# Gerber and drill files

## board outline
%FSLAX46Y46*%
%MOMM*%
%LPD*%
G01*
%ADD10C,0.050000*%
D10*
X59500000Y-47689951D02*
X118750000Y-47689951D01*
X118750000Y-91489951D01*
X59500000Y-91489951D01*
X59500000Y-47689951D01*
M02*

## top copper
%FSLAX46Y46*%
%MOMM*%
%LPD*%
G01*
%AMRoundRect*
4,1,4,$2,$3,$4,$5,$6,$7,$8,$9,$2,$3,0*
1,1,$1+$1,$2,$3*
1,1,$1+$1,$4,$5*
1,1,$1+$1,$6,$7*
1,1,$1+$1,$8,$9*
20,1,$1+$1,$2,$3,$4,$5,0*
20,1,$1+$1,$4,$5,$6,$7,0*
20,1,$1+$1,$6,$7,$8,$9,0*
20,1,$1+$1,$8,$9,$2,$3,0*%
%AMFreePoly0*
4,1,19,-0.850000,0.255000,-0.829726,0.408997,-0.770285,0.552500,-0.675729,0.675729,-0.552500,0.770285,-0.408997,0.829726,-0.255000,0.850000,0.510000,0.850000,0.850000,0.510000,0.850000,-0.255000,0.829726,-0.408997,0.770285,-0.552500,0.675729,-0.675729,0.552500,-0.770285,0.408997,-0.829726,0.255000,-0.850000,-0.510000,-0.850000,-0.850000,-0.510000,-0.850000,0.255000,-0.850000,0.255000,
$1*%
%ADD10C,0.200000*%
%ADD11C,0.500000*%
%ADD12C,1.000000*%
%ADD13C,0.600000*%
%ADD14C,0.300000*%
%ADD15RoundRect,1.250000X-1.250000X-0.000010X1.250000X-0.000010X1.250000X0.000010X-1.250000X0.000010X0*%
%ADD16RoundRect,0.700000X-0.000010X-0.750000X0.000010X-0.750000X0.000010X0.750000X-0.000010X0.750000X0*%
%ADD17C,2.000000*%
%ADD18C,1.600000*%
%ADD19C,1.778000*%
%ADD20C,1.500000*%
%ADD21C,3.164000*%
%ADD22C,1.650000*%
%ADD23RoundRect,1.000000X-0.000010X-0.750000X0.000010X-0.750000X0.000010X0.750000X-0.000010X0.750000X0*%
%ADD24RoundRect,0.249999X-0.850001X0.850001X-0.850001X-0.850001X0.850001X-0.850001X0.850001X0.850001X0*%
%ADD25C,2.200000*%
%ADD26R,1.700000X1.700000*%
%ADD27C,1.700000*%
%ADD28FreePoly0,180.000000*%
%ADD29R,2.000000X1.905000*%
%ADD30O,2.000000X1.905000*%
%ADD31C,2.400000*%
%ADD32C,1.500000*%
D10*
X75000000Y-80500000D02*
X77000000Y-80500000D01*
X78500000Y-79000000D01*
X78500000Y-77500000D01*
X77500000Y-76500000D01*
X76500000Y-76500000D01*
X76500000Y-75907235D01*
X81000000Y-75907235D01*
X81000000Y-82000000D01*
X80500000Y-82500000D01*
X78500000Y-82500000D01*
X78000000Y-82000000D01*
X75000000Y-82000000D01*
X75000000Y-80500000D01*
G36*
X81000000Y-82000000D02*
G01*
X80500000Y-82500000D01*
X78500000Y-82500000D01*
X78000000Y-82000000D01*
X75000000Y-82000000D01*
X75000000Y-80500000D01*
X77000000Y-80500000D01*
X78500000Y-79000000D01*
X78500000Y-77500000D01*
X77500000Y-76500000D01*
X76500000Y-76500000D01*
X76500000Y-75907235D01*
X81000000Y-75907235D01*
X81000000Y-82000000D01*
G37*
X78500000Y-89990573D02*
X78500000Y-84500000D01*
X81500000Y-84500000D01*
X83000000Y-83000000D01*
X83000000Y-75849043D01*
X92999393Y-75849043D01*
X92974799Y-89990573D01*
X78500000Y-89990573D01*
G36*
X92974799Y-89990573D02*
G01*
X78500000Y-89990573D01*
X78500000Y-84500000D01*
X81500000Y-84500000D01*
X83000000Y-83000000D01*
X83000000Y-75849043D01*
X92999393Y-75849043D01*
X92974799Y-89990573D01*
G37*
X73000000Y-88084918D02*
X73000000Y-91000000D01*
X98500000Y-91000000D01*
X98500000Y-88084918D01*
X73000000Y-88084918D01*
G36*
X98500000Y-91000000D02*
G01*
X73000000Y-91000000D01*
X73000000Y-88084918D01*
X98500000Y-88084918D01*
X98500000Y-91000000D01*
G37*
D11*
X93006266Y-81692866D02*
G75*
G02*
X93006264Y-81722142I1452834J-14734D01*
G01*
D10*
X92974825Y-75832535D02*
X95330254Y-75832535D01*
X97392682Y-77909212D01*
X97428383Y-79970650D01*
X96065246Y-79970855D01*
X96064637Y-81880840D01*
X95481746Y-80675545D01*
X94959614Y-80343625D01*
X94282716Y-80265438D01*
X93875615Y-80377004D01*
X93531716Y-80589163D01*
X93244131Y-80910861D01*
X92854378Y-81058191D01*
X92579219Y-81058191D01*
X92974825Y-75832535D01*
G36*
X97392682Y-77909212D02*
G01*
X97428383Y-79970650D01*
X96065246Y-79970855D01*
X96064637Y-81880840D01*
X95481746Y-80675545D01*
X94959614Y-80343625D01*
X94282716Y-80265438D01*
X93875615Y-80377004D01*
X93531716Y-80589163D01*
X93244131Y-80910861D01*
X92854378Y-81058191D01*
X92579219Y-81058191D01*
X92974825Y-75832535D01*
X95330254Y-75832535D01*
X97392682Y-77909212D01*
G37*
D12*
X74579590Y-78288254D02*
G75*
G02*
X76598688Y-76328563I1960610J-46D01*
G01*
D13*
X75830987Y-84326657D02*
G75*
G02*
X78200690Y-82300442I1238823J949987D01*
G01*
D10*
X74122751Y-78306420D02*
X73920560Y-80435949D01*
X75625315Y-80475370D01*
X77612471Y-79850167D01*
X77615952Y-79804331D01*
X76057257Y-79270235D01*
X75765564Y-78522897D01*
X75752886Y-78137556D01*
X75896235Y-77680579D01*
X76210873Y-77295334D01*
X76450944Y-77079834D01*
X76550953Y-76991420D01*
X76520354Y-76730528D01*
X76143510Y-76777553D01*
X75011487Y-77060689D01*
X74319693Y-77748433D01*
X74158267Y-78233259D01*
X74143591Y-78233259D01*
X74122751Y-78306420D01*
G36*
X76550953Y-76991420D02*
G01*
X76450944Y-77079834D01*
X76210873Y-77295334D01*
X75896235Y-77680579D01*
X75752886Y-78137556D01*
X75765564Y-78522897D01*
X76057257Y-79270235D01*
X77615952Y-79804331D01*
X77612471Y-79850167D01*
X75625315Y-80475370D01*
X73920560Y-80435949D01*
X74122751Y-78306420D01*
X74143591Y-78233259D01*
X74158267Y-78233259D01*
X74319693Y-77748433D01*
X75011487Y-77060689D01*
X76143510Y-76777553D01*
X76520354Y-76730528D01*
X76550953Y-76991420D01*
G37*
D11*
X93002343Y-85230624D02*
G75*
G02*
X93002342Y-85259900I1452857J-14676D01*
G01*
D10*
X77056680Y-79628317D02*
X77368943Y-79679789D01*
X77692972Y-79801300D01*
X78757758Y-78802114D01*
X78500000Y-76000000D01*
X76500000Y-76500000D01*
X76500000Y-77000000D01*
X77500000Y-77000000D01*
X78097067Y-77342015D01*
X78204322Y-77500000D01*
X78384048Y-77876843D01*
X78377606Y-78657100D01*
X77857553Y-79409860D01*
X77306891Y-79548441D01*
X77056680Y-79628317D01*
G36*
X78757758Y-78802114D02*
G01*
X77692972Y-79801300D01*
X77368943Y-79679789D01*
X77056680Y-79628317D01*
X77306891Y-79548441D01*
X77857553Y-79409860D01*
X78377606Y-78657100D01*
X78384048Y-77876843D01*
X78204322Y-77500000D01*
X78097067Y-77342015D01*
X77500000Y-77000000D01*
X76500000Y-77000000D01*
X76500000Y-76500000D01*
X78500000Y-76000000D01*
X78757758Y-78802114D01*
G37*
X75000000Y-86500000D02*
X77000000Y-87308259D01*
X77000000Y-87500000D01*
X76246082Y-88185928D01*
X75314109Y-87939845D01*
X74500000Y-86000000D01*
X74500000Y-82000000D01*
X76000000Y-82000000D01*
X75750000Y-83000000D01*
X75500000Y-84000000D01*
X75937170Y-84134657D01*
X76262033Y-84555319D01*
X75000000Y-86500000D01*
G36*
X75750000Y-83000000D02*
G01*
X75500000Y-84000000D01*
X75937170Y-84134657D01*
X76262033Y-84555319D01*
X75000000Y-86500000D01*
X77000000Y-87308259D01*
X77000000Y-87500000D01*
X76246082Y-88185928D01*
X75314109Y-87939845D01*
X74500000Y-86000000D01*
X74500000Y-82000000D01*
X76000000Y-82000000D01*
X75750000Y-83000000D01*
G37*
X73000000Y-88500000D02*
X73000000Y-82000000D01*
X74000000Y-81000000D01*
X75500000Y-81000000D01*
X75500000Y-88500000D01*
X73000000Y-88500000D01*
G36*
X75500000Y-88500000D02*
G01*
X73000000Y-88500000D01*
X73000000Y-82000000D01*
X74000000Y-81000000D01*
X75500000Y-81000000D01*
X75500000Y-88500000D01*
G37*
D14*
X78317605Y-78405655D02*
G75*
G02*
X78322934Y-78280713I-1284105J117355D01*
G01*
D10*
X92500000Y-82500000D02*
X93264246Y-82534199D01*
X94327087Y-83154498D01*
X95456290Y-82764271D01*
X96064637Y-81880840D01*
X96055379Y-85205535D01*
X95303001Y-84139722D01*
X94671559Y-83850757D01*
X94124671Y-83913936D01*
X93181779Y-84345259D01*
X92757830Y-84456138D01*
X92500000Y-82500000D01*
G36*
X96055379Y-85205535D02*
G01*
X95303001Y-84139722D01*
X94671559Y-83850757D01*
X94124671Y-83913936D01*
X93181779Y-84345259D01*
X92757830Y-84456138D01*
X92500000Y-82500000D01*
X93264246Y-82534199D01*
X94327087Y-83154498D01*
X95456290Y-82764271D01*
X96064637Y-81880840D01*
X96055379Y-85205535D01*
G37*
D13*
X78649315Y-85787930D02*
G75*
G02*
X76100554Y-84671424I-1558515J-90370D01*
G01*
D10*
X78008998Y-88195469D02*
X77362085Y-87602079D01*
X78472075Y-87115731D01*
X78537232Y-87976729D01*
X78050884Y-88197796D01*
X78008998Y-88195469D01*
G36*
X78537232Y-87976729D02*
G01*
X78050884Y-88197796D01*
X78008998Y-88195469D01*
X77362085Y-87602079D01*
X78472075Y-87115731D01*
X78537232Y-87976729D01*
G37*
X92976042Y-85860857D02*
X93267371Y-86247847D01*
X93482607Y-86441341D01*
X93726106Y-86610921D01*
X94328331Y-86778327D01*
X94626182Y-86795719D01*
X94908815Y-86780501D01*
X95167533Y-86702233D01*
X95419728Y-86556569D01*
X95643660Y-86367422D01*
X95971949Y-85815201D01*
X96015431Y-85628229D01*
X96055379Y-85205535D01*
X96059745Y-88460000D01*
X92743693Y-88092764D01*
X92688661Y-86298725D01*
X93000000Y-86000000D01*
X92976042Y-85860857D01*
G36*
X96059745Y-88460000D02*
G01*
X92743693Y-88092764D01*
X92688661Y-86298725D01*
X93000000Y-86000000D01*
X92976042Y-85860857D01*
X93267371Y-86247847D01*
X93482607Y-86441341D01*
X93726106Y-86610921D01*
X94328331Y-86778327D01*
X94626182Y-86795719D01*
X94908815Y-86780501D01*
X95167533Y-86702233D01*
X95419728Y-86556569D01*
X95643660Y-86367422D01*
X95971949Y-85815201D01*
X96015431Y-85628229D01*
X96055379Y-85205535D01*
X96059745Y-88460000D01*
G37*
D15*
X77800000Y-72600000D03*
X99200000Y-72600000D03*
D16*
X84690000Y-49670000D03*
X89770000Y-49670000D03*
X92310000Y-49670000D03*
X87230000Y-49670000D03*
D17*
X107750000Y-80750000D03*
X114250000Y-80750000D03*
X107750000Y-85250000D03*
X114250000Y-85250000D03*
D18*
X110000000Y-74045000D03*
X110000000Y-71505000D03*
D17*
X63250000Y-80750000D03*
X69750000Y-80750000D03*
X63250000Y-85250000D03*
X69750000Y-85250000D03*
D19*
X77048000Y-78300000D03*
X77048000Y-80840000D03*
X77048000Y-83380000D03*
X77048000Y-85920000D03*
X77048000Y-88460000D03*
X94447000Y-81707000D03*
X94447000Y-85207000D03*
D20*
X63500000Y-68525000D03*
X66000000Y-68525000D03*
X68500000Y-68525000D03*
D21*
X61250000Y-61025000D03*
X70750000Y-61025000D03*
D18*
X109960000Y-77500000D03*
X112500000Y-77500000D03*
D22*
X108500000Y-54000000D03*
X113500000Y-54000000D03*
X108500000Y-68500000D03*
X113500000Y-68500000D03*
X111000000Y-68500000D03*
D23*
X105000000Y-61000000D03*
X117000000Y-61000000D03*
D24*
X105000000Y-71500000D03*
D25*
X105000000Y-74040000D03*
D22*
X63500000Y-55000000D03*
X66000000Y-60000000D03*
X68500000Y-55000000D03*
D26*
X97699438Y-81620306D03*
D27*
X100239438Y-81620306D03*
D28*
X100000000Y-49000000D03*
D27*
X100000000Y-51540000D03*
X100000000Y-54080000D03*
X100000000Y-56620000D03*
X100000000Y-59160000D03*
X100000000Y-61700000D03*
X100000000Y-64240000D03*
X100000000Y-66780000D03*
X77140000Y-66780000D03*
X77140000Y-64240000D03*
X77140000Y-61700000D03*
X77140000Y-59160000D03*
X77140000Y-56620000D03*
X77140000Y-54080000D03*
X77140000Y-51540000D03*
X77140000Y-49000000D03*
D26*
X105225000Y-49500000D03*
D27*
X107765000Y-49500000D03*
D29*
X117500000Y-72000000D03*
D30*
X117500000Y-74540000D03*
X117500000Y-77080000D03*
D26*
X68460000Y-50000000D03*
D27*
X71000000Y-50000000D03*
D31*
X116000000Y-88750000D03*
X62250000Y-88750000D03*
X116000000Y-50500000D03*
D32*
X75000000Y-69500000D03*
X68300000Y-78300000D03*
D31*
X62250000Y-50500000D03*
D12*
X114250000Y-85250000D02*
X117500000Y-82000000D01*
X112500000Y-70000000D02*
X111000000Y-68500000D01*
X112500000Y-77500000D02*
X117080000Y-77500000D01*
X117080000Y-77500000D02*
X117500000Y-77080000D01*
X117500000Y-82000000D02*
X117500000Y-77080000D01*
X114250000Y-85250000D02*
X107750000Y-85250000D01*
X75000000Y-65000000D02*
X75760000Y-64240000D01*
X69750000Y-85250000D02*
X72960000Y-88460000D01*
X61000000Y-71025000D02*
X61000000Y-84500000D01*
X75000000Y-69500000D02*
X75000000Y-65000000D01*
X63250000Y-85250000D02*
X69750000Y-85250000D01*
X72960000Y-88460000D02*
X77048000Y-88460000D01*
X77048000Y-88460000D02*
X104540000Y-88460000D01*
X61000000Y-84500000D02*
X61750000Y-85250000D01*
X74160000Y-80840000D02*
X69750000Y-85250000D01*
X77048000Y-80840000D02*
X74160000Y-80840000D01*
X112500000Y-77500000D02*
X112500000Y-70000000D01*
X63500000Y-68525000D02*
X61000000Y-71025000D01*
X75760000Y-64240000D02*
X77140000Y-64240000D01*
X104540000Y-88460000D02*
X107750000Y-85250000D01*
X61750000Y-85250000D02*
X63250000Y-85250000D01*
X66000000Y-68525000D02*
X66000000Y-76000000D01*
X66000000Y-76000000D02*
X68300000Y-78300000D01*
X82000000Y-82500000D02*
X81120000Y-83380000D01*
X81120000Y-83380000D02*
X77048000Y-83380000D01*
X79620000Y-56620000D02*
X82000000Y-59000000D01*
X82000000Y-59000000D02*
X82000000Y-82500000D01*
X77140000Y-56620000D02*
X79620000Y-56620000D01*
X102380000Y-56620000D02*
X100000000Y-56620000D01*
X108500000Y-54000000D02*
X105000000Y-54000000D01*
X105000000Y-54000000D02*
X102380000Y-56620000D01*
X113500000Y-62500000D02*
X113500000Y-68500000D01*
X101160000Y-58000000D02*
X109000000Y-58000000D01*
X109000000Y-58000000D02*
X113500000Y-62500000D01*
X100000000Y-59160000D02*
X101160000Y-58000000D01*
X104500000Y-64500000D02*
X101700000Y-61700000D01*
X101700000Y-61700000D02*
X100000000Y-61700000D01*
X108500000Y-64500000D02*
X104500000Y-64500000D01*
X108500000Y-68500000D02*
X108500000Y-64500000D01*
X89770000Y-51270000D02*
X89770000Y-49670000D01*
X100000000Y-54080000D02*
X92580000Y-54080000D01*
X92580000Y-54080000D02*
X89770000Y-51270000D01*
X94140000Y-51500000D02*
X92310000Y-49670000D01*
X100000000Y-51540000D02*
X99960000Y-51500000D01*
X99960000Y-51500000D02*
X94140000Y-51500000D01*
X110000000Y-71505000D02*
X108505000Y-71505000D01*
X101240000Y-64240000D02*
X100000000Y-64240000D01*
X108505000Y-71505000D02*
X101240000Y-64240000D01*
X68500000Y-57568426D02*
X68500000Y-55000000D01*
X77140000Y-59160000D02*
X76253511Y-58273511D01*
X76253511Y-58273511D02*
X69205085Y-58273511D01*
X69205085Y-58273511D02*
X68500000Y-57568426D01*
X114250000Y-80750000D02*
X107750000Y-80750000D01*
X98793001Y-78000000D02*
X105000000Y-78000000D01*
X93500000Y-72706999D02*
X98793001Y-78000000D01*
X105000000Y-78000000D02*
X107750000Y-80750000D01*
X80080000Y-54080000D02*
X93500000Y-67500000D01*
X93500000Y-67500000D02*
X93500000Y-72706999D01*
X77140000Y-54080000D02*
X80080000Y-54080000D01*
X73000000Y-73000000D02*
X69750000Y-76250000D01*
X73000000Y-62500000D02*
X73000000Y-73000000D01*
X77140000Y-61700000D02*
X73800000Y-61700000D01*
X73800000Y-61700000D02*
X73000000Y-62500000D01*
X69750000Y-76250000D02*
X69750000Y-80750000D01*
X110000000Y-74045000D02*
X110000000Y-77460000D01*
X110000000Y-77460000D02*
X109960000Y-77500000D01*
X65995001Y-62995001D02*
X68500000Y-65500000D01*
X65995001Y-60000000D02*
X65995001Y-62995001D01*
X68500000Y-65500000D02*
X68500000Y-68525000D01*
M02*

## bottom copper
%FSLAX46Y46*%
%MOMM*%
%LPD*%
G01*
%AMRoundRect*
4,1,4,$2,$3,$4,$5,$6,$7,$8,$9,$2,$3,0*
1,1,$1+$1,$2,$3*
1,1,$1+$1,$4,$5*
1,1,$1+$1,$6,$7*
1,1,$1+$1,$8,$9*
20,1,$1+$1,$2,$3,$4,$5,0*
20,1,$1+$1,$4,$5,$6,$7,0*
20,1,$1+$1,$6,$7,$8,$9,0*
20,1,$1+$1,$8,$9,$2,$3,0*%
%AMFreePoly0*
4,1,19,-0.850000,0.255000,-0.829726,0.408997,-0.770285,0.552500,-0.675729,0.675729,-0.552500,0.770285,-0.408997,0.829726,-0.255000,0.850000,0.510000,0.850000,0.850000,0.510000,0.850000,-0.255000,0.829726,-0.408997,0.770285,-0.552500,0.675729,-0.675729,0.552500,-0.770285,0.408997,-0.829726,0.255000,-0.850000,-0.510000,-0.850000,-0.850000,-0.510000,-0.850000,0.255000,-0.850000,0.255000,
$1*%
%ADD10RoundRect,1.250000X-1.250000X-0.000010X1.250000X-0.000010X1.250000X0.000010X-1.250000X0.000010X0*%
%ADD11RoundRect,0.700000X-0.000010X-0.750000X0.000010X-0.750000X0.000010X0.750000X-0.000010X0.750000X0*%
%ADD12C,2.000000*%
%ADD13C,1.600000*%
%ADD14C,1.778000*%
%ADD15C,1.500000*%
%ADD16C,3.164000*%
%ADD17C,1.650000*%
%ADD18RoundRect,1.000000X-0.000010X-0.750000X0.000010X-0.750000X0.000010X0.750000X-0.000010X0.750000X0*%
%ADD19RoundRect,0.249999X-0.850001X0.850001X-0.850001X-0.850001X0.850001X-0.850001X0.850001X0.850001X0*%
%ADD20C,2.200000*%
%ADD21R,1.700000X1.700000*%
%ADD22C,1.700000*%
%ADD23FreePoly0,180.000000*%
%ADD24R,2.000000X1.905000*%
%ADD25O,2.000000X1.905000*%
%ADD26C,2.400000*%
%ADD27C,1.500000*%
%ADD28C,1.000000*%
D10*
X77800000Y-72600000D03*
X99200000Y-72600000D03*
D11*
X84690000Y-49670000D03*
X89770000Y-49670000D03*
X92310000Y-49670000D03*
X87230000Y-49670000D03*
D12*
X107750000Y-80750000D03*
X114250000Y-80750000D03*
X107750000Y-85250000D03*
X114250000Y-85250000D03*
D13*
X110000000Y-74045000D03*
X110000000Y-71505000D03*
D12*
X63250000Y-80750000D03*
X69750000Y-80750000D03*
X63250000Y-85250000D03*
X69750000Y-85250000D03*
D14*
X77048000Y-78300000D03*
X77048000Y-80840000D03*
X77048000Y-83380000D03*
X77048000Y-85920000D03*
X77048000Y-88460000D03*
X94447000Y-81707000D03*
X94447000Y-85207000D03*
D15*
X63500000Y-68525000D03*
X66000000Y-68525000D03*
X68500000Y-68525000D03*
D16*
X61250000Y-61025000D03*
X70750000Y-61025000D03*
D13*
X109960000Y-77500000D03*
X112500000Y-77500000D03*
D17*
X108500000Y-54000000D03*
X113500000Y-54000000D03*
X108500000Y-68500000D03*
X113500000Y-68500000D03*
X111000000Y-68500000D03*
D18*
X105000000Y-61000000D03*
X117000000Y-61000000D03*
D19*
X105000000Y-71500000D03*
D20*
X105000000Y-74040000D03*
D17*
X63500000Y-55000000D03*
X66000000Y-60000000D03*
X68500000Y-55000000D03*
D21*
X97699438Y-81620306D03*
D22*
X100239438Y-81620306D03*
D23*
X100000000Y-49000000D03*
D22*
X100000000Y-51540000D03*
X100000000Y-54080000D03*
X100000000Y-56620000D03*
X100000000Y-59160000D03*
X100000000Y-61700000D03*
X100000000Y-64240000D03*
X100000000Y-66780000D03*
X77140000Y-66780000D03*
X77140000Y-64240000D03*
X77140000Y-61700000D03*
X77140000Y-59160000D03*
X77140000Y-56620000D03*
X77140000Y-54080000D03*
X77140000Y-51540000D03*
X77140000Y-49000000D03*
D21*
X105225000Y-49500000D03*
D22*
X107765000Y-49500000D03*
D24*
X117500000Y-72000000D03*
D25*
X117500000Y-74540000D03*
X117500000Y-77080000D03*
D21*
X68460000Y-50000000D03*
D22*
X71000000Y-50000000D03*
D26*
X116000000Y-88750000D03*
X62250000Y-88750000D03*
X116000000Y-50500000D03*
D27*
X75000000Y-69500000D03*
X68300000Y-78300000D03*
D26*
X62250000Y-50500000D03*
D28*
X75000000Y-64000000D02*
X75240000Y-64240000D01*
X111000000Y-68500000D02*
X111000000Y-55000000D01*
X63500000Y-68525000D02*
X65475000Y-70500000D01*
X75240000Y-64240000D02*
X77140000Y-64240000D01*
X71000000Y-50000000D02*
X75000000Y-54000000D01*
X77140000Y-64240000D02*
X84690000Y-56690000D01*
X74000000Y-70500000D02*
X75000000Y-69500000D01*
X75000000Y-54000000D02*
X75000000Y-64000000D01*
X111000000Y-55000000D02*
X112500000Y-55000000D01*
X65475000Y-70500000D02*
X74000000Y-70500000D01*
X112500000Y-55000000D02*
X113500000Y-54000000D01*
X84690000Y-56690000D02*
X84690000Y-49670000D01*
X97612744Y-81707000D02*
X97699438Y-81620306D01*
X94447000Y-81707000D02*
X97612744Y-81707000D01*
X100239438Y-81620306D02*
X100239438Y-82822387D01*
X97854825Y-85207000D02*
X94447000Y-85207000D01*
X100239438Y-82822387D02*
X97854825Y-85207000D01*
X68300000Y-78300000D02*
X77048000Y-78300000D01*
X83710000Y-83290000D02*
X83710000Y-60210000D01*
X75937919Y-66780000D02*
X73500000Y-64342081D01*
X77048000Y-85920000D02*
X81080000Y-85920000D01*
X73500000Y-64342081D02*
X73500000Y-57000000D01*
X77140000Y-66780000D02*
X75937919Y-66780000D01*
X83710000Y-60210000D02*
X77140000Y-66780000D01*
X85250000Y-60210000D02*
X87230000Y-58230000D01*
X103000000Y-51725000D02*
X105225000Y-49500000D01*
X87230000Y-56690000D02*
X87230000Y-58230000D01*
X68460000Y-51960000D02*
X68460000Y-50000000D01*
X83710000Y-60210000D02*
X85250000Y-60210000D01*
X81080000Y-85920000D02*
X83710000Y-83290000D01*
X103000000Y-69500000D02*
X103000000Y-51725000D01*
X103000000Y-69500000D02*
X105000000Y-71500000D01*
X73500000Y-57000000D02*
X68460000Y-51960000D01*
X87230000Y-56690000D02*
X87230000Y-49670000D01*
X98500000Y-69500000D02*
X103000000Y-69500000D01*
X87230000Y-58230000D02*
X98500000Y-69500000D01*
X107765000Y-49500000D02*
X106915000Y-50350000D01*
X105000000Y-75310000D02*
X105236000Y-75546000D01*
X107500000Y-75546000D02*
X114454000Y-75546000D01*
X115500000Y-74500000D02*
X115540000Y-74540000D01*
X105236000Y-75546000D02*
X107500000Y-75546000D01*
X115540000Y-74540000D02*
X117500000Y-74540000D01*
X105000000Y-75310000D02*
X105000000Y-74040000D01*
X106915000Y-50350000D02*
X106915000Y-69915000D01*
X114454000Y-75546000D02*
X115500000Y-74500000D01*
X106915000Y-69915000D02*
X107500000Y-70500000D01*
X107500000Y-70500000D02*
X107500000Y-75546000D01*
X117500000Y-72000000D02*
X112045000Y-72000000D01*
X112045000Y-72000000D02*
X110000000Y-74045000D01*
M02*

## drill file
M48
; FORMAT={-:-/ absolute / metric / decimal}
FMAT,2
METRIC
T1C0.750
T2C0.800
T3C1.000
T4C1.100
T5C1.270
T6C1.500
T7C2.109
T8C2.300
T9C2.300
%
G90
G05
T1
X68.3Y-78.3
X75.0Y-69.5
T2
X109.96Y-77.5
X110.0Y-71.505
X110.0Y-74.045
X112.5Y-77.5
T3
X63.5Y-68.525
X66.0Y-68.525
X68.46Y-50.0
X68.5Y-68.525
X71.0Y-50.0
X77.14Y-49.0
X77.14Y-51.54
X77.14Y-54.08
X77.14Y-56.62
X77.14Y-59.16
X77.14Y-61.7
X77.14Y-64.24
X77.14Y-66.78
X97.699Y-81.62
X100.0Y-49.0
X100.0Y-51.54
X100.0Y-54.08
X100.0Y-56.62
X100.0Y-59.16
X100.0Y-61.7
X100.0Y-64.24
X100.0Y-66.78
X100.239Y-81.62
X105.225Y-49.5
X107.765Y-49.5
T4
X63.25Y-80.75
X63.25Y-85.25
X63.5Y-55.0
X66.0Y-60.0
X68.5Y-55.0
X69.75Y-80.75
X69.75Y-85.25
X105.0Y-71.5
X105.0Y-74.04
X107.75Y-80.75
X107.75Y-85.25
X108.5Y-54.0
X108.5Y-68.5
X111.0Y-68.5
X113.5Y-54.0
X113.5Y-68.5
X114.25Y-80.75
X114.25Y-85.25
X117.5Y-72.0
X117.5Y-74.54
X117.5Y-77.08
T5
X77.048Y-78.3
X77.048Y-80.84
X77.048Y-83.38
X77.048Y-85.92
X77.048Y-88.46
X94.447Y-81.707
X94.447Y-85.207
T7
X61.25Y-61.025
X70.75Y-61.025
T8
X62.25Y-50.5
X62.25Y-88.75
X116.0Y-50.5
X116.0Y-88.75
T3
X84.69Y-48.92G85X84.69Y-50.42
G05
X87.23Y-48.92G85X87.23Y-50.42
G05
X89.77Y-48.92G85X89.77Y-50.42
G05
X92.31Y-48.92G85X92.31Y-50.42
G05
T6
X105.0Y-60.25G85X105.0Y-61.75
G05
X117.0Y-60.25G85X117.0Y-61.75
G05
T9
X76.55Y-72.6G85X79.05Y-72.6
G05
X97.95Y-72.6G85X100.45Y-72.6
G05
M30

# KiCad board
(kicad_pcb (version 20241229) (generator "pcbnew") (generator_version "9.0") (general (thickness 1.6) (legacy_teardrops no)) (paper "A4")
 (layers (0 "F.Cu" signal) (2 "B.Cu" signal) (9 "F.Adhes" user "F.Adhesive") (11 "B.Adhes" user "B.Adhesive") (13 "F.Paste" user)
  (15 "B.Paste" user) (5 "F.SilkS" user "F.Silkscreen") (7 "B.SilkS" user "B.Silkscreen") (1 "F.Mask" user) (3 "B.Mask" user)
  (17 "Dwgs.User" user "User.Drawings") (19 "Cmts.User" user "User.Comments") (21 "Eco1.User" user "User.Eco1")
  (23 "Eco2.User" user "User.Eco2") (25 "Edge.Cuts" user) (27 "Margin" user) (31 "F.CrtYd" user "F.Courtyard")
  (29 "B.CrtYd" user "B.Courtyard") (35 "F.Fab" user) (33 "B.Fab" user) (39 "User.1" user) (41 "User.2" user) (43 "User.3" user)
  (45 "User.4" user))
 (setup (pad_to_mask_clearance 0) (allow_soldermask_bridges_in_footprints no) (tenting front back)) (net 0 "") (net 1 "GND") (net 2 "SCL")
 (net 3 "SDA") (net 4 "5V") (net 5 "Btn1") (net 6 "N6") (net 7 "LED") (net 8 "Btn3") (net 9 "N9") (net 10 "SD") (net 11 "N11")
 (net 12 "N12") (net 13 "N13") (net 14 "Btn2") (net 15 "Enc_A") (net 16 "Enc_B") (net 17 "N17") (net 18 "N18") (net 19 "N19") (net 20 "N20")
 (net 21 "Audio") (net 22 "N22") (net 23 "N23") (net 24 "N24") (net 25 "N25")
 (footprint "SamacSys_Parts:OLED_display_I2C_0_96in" (layer "F.Cu") (at 88.5 61.5)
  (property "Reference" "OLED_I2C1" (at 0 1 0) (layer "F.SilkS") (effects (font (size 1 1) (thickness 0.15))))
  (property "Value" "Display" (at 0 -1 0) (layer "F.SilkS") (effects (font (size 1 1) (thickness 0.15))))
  (pad "" np_thru_hole roundrect (at -10.7 11.1) (size 5 2.5) (drill oval 4.8 2.3) (layers "*.Cu" "*.Mask") (roundrect_rratio 0.5))
  (pad "" np_thru_hole roundrect (at 10.7 11.1) (size 5 2.5) (drill oval 4.8 2.3) (layers "*.Cu" "*.Mask") (roundrect_rratio 0.5))
  (pad "GND" thru_hole roundrect (at -3.81 -11.83) (size 1.4 2.9) (drill oval 1 2.5) (layers "*.Cu" "*.Mask") (remove_unused_layers no)
   (roundrect_rratio 0.5) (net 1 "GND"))
  (pad "SCL" thru_hole roundrect (at 1.27 -11.83) (size 1.4 2.9) (drill oval 1 2.5) (layers "*.Cu" "*.Mask") (remove_unused_layers no)
   (roundrect_rratio 0.5) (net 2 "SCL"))
  (pad "SDA" thru_hole roundrect (at 3.81 -11.83) (size 1.4 2.9) (drill oval 1 2.5) (layers "*.Cu" "*.Mask") (remove_unused_layers no)
   (roundrect_rratio 0.5) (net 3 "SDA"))
  (pad "Vcc" thru_hole roundrect (at -1.27 -11.83) (size 1.4 2.9) (drill oval 1 2.5) (layers "*.Cu" "*.Mask") (remove_unused_layers no)
   (roundrect_rratio 0.5) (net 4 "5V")))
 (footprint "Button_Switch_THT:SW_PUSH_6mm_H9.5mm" (layer "F.Cu") (at 107.75 80.75)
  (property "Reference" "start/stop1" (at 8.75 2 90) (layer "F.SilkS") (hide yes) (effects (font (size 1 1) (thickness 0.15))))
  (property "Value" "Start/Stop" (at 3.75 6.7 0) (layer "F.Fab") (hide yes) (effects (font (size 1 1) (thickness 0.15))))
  (pad "1" thru_hole circle (at 0 0 90) (size 2 2) (drill 1.1) (layers "*.Cu" "*.Mask") (remove_unused_layers no) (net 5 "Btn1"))
  (pad "1" thru_hole circle (at 6.5 0 90) (size 2 2) (drill 1.1) (layers "*.Cu" "*.Mask") (remove_unused_layers no) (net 5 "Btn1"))
  (pad "2" thru_hole circle (at 0 4.5 90) (size 2 2) (drill 1.1) (layers "*.Cu" "*.Mask") (remove_unused_layers no) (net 1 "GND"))
  (pad "2" thru_hole circle (at 6.5 4.5 90) (size 2 2) (drill 1.1) (layers "*.Cu" "*.Mask") (remove_unused_layers no) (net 1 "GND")))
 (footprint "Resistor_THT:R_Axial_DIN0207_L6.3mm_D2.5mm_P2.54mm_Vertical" (layer "F.Cu") (at 110 74.045 90)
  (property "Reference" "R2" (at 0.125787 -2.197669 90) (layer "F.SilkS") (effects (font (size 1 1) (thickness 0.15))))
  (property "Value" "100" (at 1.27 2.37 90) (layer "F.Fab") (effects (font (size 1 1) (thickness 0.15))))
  (pad "1" thru_hole circle (at 0 0 90) (size 1.6 1.6) (drill 0.8) (layers "*.Cu" "*.Mask") (remove_unused_layers no) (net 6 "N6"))
  (pad "2" thru_hole circle (at 2.54 0 90) (size 1.6 1.6) (drill 0.8) (layers "*.Cu" "*.Mask") (remove_unused_layers no) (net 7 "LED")))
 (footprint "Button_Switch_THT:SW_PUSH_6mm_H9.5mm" (layer "F.Cu") (at 63.25 80.75)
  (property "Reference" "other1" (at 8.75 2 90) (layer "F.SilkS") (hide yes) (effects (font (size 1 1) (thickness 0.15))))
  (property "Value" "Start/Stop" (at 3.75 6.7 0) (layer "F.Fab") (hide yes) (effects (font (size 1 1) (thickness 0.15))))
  (pad "1" thru_hole circle (at 0 0 90) (size 2 2) (drill 1.1) (layers "*.Cu" "*.Mask") (remove_unused_layers no) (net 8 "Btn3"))
  (pad "1" thru_hole circle (at 6.5 0 90) (size 2 2) (drill 1.1) (layers "*.Cu" "*.Mask") (remove_unused_layers no) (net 8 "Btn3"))
  (pad "2" thru_hole circle (at 0 4.5 90) (size 2 2) (drill 1.1) (layers "*.Cu" "*.Mask") (remove_unused_layers no) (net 1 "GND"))
  (pad "2" thru_hole circle (at 6.5 4.5 90) (size 2 2) (drill 1.1) (layers "*.Cu" "*.Mask") (remove_unused_layers no) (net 1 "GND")))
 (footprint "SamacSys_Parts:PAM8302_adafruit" (layer "F.Cu") (at 74 91)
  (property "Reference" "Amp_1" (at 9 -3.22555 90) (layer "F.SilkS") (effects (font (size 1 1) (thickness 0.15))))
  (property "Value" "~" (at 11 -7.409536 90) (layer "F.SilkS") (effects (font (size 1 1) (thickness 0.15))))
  (pad "1" thru_hole circle (at 3.048 -12.7) (size 1.778 1.778) (drill 1.27) (layers "*.Cu" "*.Mask") (remove_unused_layers no) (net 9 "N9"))
  (pad "2" thru_hole circle (at 3.048 -10.16) (size 1.778 1.778) (drill 1.27) (layers "*.Cu" "*.Mask") (remove_unused_layers no)
   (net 1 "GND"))
  (pad "3" thru_hole circle (at 3.048 -7.62) (size 1.778 1.778) (drill 1.27) (layers "*.Cu" "*.Mask") (remove_unused_layers no)
   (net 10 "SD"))
  (pad "4" thru_hole circle (at 3.048 -5.08) (size 1.778 1.778) (drill 1.27) (layers "*.Cu" "*.Mask") (remove_unused_layers no) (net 4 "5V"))
  (pad "5" thru_hole circle (at 3.048 -2.54) (size 1.778 1.778) (drill 1.27) (layers "*.Cu" "*.Mask") (remove_unused_layers no)
   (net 1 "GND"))
  (pad "6" thru_hole circle (at 20.447 -9.293) (size 1.778 1.778) (drill 1.27) (layers "*.Cu" "*.Mask") (remove_unused_layers no)
   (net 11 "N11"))
  (pad "7" thru_hole circle (at 20.447 -5.793) (size 1.778 1.778) (drill 1.27) (layers "*.Cu" "*.Mask") (remove_unused_layers no)
   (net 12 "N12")))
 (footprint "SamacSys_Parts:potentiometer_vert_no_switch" (layer "F.Cu") (at 66 63)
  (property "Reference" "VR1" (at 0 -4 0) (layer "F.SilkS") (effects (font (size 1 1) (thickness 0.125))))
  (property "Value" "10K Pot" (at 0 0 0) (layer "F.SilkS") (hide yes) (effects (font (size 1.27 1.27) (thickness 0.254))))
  (pad "1" thru_hole circle (at -2.5 5.525) (size 1.5 1.5) (drill 1) (layers "*.Cu" "*.Mask") (remove_unused_layers no) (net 1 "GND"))
  (pad "2" thru_hole circle (at 0 5.525) (size 1.5 1.5) (drill 1) (layers "*.Cu" "*.Mask") (remove_unused_layers no) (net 9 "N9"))
  (pad "3" thru_hole circle (at 2.5 5.525) (size 1.5 1.5) (drill 1) (layers "*.Cu" "*.Mask") (remove_unused_layers no) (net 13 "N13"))
  (pad "MH1" thru_hole circle (at -4.75 -1.975) (size 3.164 3.164) (drill 2.1095) (layers "*.Cu" "*.Mask") (remove_unused_layers no))
  (pad "MH2" thru_hole circle (at 4.75 -1.975) (size 3.164 3.164) (drill 2.1095) (layers "*.Cu" "*.Mask") (remove_unused_layers no)))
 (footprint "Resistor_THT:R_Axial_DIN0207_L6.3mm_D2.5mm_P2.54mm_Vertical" (layer "F.Cu") (at 109.96 77.5)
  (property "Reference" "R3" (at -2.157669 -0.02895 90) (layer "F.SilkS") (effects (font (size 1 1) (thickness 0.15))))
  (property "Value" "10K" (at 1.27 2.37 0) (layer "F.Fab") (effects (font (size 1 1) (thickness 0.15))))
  (pad "1" thru_hole circle (at 0 0) (size 1.6 1.6) (drill 0.8) (layers "*.Cu" "*.Mask") (remove_unused_layers no) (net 6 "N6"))
  (pad "2" thru_hole circle (at 2.54 0) (size 1.6 1.6) (drill 0.8) (layers "*.Cu" "*.Mask") (remove_unused_layers no) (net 1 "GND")))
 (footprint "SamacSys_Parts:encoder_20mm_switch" (layer "F.Cu") (at 108.5 54)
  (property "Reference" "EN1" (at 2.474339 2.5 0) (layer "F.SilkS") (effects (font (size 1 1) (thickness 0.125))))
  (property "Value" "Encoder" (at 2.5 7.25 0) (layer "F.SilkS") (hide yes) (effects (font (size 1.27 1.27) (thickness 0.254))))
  (pad "1" thru_hole circle (at 0 0) (size 1.65 1.65) (drill 1.1) (layers "*.Cu" "*.Mask") (remove_unused_layers no) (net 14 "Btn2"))
  (pad "2" thru_hole circle (at 5 0) (size 1.65 1.65) (drill 1.1) (layers "*.Cu" "*.Mask") (remove_unused_layers no) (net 1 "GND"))
  (pad "A1" thru_hole circle (at 0 14.5) (size 1.65 1.65) (drill 1.1) (layers "*.Cu" "*.Mask") (remove_unused_layers no) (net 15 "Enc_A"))
  (pad "B1" thru_hole circle (at 5 14.5) (size 1.65 1.65) (drill 1.1) (layers "*.Cu" "*.Mask") (remove_unused_layers no) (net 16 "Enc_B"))
  (pad "GND" thru_hole circle (at 2.5 14.5) (size 1.65 1.65) (drill 1.1) (layers "*.Cu" "*.Mask") (remove_unused_layers no) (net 1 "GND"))
  (pad "MH1" thru_hole roundrect (at -3.5 7) (size 2 3.5) (drill oval 1.5 3) (layers "*.Cu" "*.Mask") (remove_unused_layers no)
   (roundrect_rratio 0.5) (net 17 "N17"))
  (pad "MH2" thru_hole roundrect (at 8.5 7) (size 2 3.5) (drill oval 1.5 3) (layers "*.Cu" "*.Mask") (remove_unused_layers no)
   (roundrect_rratio 0.5) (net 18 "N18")))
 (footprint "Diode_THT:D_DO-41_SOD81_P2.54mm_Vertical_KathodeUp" (layer "F.Cu") (at 105 71.5 -90)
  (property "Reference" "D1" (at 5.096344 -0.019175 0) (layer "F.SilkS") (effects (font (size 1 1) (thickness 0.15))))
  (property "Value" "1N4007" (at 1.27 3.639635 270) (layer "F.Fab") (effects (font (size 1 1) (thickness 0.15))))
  (pad "1" thru_hole roundrect (at 0 0 270) (size 2.2 2.2) (drill 1.1) (layers "*.Cu" "*.Mask") (remove_unused_layers no)
   (roundrect_rratio 0.113636) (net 4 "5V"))
  (pad "2" thru_hole circle (at 2.54 0 270) (size 2.2 2.2) (drill 1.1) (layers "*.Cu" "*.Mask") (remove_unused_layers no) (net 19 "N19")))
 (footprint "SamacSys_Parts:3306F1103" (layer "B.Cu") (at 66 57.5)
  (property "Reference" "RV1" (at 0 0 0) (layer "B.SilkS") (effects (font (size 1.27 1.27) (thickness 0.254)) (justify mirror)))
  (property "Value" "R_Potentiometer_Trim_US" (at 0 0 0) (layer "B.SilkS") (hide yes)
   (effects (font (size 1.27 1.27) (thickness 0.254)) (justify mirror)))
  (pad "1" thru_hole circle (at -2.5 -2.5) (size 1.65 1.65) (drill 1.1) (layers "*.Cu" "*.Mask") (remove_unused_layers no) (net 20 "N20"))
  (pad "2" thru_hole circle (at 0 2.5) (size 1.65 1.65) (drill 1.1) (layers "*.Cu" "*.Mask") (remove_unused_layers no) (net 13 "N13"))
  (pad "3" thru_hole circle (at 2.5 -2.5) (size 1.65 1.65) (drill 1.1) (layers "*.Cu" "*.Mask") (remove_unused_layers no) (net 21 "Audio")))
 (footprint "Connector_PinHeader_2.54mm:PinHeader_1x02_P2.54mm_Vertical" (layer "B.Cu") (at 97.699438 81.620306 -90)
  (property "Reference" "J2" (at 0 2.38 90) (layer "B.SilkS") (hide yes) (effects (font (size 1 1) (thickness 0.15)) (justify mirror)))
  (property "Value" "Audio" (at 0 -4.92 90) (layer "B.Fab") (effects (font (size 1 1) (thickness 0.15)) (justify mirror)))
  (pad "1" thru_hole rect (at 0 0 270) (size 1.7 1.7) (drill 1) (layers "*.Cu" "*.Mask") (remove_unused_layers no) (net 11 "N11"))
  (pad "2" thru_hole circle (at 0 -2.54 270) (size 1.7 1.7) (drill 1) (layers "*.Cu" "*.Mask") (remove_unused_layers no) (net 12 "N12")))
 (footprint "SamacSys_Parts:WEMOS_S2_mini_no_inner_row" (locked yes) (layer "B.Cu") (at 100 49 180)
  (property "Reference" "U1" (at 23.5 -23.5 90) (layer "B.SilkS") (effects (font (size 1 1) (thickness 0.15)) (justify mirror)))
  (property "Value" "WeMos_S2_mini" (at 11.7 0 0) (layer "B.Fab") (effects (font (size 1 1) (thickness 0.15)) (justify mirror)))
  (pad "1" thru_hole roundrect (at 0 0 180) (size 1.7 1.7) (drill 1) (layers "*.Cu" "*.Mask") (remove_unused_layers no)
   (roundrect_rratio 0.35) (chamfer_ratio 0.2) (chamfer top_right bottom_left) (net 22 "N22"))
  (pad "2" thru_hole circle (at 0 -2.54 180) (size 1.7 1.7) (drill 1) (layers "*.Cu" "*.Mask") (remove_unused_layers no) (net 3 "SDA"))
  (pad "3" thru_hole circle (at 0 -5.08 180) (size 1.7 1.7) (drill 1) (layers "*.Cu" "*.Mask") (remove_unused_layers no) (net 2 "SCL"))
  (pad "4" thru_hole circle (at 0 -7.62 180) (size 1.7 1.7) (drill 1) (layers "*.Cu" "*.Mask") (remove_unused_layers no) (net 14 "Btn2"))
  (pad "5" thru_hole circle (at 0 -10.16 180) (size 1.7 1.7) (drill 1) (layers "*.Cu" "*.Mask") (remove_unused_layers no) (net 16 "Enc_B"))
  (pad "6" thru_hole circle (at 0 -12.7 180) (size 1.7 1.7) (drill 1) (layers "*.Cu" "*.Mask") (remove_unused_layers no) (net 15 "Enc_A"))
  (pad "7" thru_hole circle (at 0 -15.24 180) (size 1.7 1.7) (drill 1) (layers "*.Cu" "*.Mask") (remove_unused_layers no) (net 7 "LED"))
  (pad "8" thru_hole circle (at 0 -17.78 180) (size 1.7 1.7) (drill 1) (layers "*.Cu" "*.Mask") (remove_unused_layers no) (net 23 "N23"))
  (pad "9" thru_hole circle (at 22.86 -17.78 180) (size 1.7 1.7) (drill 1) (layers "*.Cu" "*.Mask") (remove_unused_layers no) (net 4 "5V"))
  (pad "10" thru_hole circle (at 22.86 -15.24 180) (size 1.7 1.7) (drill 1) (layers "*.Cu" "*.Mask") (remove_unused_layers no) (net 1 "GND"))
  (pad "11" thru_hole circle (at 22.86 -12.7 180) (size 1.7 1.7) (drill 1) (layers "*.Cu" "*.Mask") (remove_unused_layers no) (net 8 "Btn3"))
  (pad "12" thru_hole circle (at 22.86 -10.16 180) (size 1.7 1.7) (drill 1) (layers "*.Cu" "*.Mask") (remove_unused_layers no)
   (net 21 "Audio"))
  (pad "13" thru_hole circle (at 22.86 -7.62 180) (size 1.7 1.7) (drill 1) (layers "*.Cu" "*.Mask") (remove_unused_layers no) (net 10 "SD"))
  (pad "14" thru_hole circle (at 22.86 -5.08 180) (size 1.7 1.7) (drill 1) (layers "*.Cu" "*.Mask") (remove_unused_layers no) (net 5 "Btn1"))
  (pad "15" thru_hole circle (at 22.86 -2.54 180) (size 1.7 1.7) (drill 1) (layers "*.Cu" "*.Mask") (remove_unused_layers no) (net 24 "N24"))
  (pad "16" thru_hole circle (at 22.86 0 180) (size 1.7 1.7) (drill 1) (layers "*.Cu" "*.Mask") (remove_unused_layers no) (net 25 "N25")))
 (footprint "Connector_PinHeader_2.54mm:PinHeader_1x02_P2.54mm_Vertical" (layer "B.Cu") (at 105.225 49.5 -90)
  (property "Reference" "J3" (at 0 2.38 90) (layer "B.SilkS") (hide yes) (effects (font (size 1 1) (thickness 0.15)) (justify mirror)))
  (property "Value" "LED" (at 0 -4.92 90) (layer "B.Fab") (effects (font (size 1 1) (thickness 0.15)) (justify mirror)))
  (pad "1" thru_hole rect (at 0 0 270) (size 1.7 1.7) (drill 1) (layers "*.Cu" "*.Mask") (remove_unused_layers no) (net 4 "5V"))
  (pad "2" thru_hole circle (at 0 -2.54 270) (size 1.7 1.7) (drill 1) (layers "*.Cu" "*.Mask") (remove_unused_layers no) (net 19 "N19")))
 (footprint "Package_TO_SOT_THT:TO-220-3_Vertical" (layer "B.Cu") (at 117.5 72 -90)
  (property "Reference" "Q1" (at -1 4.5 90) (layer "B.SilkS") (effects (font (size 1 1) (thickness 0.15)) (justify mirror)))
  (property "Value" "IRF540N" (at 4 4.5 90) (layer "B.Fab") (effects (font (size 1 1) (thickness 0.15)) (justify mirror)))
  (pad "1" thru_hole rect (at 0 0 270) (size 1.905 2) (drill 1.1) (layers "*.Cu" "*.Mask") (remove_unused_layers no) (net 6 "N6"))
  (pad "2" thru_hole oval (at 2.54 0 270) (size 1.905 2) (drill 1.1) (layers "*.Cu" "*.Mask") (remove_unused_layers no) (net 19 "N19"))
  (pad "3" thru_hole oval (at 5.08 0 270) (size 1.905 2) (drill 1.1) (layers "*.Cu" "*.Mask") (remove_unused_layers no) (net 1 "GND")))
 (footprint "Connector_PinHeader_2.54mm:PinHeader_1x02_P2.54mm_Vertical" (layer "B.Cu") (at 68.46 50 -90)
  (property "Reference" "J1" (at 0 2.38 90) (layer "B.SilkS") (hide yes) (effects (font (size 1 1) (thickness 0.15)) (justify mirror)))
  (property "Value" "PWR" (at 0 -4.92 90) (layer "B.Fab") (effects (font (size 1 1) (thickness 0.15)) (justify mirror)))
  (pad "1" thru_hole rect (at 0 0 270) (size 1.7 1.7) (drill 1) (layers "*.Cu" "*.Mask") (remove_unused_layers no) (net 4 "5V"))
  (pad "2" thru_hole circle (at 0 -2.54 270) (size 1.7 1.7) (drill 1) (layers "*.Cu" "*.Mask") (remove_unused_layers no) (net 1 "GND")))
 (gr_poly
  (pts (xy 75 80.5) (xy 77 80.5) (xy 78.5 79) (xy 78.5 77.5) (xy 77.5 76.5) (xy 76.5 76.5) (xy 76.5 75.907235) (xy 81 75.907235) (xy 81 82)
   (xy 80.5 82.5) (xy 78.5 82.5) (xy 78 82) (xy 75 82))
  (stroke (width 0.2) (type solid)) (fill yes) (layer "F.Cu") (net 1))
 (gr_poly
  (pts (xy 78.5 89.990573) (xy 78.5 84.5) (xy 81.5 84.5) (xy 83 83) (xy 83 75.849043) (xy 92.999393 75.849043) (xy 92.974799 89.990573))
  (stroke (width 0.2) (type solid)) (fill yes) (layer "F.Cu") (net 1))
 (gr_poly
  (pts (xy 73 88.084918) (xy 73 91) (xy 98.5 91) (xy 98.5 88.084918)) (stroke (width 0.2) (type solid)) (fill yes) (layer "F.Cu") (net 1))
 (gr_arc (start 93.006266 81.692866) (mid 95.912022 81.707578) (end 93.006265 81.722142) (stroke (width 0.5) (type solid)) (layer "F.Cu")
  (net 1))
 (gr_poly
  (pts (xy 92.974825 75.832535) (xy 95.330254 75.832535) (xy 97.392682 77.909212) (xy 97.428383 79.97065) (xy 96.065246 79.970855)
   (xy 96.064637 81.88084) (xy 95.481746 80.675545) (xy 94.959614 80.343625) (xy 94.282716 80.265438) (xy 93.875615 80.377004)
   (xy 93.531716 80.589163) (xy 93.244131 80.910861) (xy 92.854378 81.058191) (xy 92.579219 81.058191))
  (stroke (width 0.2) (type solid)) (fill yes) (layer "F.Cu") (net 1))
 (gr_arc (start 74.57959 78.288254) (mid 75.174676 76.881374) (end 76.598689 76.328539) (stroke (width 1) (type solid)) (layer "F.Cu")
  (net 1))
 (gr_arc (start 75.830987 84.326657) (mid 76.055264 82.190134) (end 78.200693 82.300439) (stroke (width 0.6) (type solid)) (layer "F.Cu")
  (net 1))
 (gr_poly
  (pts (xy 74.122751 78.30642) (xy 73.92056 80.435949) (xy 75.625315 80.47537) (xy 77.612471 79.850167) (xy 77.615952 79.804331)
   (xy 76.057257 79.270235) (xy 75.765564 78.522897) (xy 75.752886 78.137556) (xy 75.896235 77.680579) (xy 76.210873 77.295334)
   (xy 76.450944 77.079834) (xy 76.550953 76.99142) (xy 76.520354 76.730528) (xy 76.14351 76.777553) (xy 75.011487 77.060689)
   (xy 74.319693 77.748433) (xy 74.158267 78.233259) (xy 74.143591 78.233259))
  (stroke (width 0.2) (type solid)) (fill yes) (layer "F.Cu") (net 1))
 (gr_arc (start 93.002343 85.230624) (mid 95.908099 85.245336) (end 93.002342 85.2599) (stroke (width 0.5) (type solid)) (layer "F.Cu")
  (net 1))
 (gr_poly
  (pts (xy 77.05668 79.628317) (xy 77.368943 79.679789) (xy 77.692972 79.8013) (xy 78.757758 78.802114) (xy 78.5 76) (xy 76.5 76.5)
   (xy 76.5 77) (xy 77.5 77) (xy 78.097067 77.342015) (xy 78.204322 77.5) (xy 78.384048 77.876843) (xy 78.377606 78.6571)
   (xy 77.857553 79.40986) (xy 77.306891 79.548441))
  (stroke (width 0.2) (type solid)) (fill yes) (layer "F.Cu") (net 1))
 (gr_poly
  (pts (xy 75 86.5) (xy 77 87.308259) (xy 77 87.5) (xy 76.246082 88.185928) (xy 75.314109 87.939845) (xy 74.5 86) (xy 74.5 82) (xy 76 82)
   (xy 75.75 83) (xy 75.5 84) (xy 75.93717 84.134657) (xy 76.262033 84.555319))
  (stroke (width 0.2) (type solid)) (fill yes) (layer "F.Cu") (net 1))
 (gr_poly
  (pts (xy 73 88.5) (xy 73 82) (xy 74 81) (xy 75.5 81) (xy 75.5 88.5)) (stroke (width 0.2) (type solid)) (fill yes) (layer "F.Cu") (net 1))
 (gr_arc (start 78.317605 78.405655) (mid 75.745269 78.233259) (end 78.322939 78.280713) (stroke (width 0.3) (type solid)) (layer "F.Cu")
  (net 1))
 (gr_poly
  (pts (xy 92.5 82.5) (xy 93.264246 82.534199) (xy 94.327087 83.154498) (xy 95.45629 82.764271) (xy 96.064637 81.88084)
   (xy 96.055379 85.205535) (xy 95.303001 84.139722) (xy 94.671559 83.850757) (xy 94.124671 83.913936) (xy 93.181779 84.345259)
   (xy 92.75783 84.456138))
  (stroke (width 0.2) (type solid)) (fill yes) (layer "F.Cu") (net 1))
 (gr_arc (start 78.649315 85.78793) (mid 76.464383 87.308259) (end 76.100546 84.671414) (stroke (width 0.6) (type solid)) (layer "F.Cu")
  (net 1))
 (gr_poly
  (pts (xy 78.008998 88.195469) (xy 77.362085 87.602079) (xy 78.472075 87.115731) (xy 78.537232 87.976729) (xy 78.050884 88.197796))
  (stroke (width 0.2) (type solid)) (fill yes) (layer "F.Cu") (net 1))
 (gr_poly
  (pts (xy 92.976042 85.860857) (xy 93.267371 86.247847) (xy 93.482607 86.441341) (xy 93.726106 86.610921) (xy 94.328331 86.778327)
   (xy 94.626182 86.795719) (xy 94.908815 86.780501) (xy 95.167533 86.702233) (xy 95.419728 86.556569) (xy 95.64366 86.367422)
   (xy 95.971949 85.815201) (xy 96.015431 85.628229) (xy 96.055379 85.205535) (xy 96.059745 88.46) (xy 92.743693 88.092764)
   (xy 92.688661 86.298725) (xy 93 86))
  (stroke (width 0.2) (type solid)) (fill yes) (layer "F.Cu") (net 1))
 (gr_rect (start 59.5 47.689951) (end 118.75 91.489951) (stroke (width 0.05) (type solid)) (fill no) (layer "Edge.Cuts"))
 (via (at 116 88.75) (size 2.4) (drill 2.3) (layers "F.Cu" "B.Cu") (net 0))
 (via (at 62.25 88.75) (size 2.4) (drill 2.3) (layers "F.Cu" "B.Cu") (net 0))
 (via (at 116 50.5) (size 2.4) (drill 2.3) (layers "F.Cu" "B.Cu") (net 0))
 (segment (start 114.25 85.25) (end 117.5 82) (width 1) (layer "F.Cu") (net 1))
 (segment (start 112.5 70) (end 111 68.5) (width 1) (layer "F.Cu") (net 1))
 (segment (start 112.5 77.5) (end 117.08 77.5) (width 1) (layer "F.Cu") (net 1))
 (segment (start 117.08 77.5) (end 117.5 77.08) (width 1) (layer "F.Cu") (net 1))
 (segment (start 117.5 82) (end 117.5 77.08) (width 1) (layer "F.Cu") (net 1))
 (segment (start 114.25 85.25) (end 107.75 85.25) (width 1) (layer "F.Cu") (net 1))
 (segment (start 75 65) (end 75.76 64.24) (width 1) (layer "F.Cu") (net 1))
 (segment (start 69.75 85.25) (end 72.96 88.46) (width 1) (layer "F.Cu") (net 1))
 (segment (start 61 71.025) (end 61 84.5) (width 1) (layer "F.Cu") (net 1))
 (segment (start 75 69.5) (end 75 65) (width 1) (layer "F.Cu") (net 1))
 (segment (start 63.25 85.25) (end 69.75 85.25) (width 1) (layer "F.Cu") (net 1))
 (segment (start 72.96 88.46) (end 77.048 88.46) (width 1) (layer "F.Cu") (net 1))
 (segment (start 77.048 88.46) (end 104.54 88.46) (width 1) (layer "F.Cu") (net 1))
 (segment (start 61 84.5) (end 61.75 85.25) (width 1) (layer "F.Cu") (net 1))
 (segment (start 74.16 80.84) (end 69.75 85.25) (width 1) (layer "F.Cu") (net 1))
 (segment (start 77.048 80.84) (end 74.16 80.84) (width 1) (layer "F.Cu") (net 1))
 (segment (start 112.5 77.5) (end 112.5 70) (width 1) (layer "F.Cu") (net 1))
 (segment (start 63.5 68.525) (end 61 71.025) (width 1) (layer "F.Cu") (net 1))
 (segment (start 75.76 64.24) (end 77.14 64.24) (width 1) (layer "F.Cu") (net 1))
 (segment (start 104.54 88.46) (end 107.75 85.25) (width 1) (layer "F.Cu") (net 1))
 (segment (start 61.75 85.25) (end 63.25 85.25) (width 1) (layer "F.Cu") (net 1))
 (via (at 75 69.5) (size 1.5) (drill 0.75) (layers "F.Cu" "B.Cu") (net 1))
 (segment (start 75 64) (end 75.24 64.24) (width 1) (layer "B.Cu") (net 1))
 (segment (start 111 68.5) (end 111 55) (width 1) (layer "B.Cu") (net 1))
 (segment (start 63.5 68.525) (end 65.475 70.5) (width 1) (layer "B.Cu") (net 1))
 (segment (start 75.24 64.24) (end 77.14 64.24) (width 1) (layer "B.Cu") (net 1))
 (segment (start 71 50) (end 75 54) (width 1) (layer "B.Cu") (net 1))
 (segment (start 77.14 64.24) (end 84.69 56.69) (width 1) (layer "B.Cu") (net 1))
 (segment (start 74 70.5) (end 75 69.5) (width 1) (layer "B.Cu") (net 1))
 (segment (start 75 54) (end 75 64) (width 1) (layer "B.Cu") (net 1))
 (segment (start 111 55) (end 112.5 55) (width 1) (layer "B.Cu") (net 1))
 (segment (start 65.475 70.5) (end 74 70.5) (width 1) (layer "B.Cu") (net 1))
 (segment (start 112.5 55) (end 113.5 54) (width 1) (layer "B.Cu") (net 1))
 (segment (start 84.69 56.69) (end 84.69 49.67) (width 1) (layer "B.Cu") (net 1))
 (segment (start 97.612744 81.707) (end 97.699438 81.620306) (width 1) (layer "B.Cu") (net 11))
 (segment (start 94.447 81.707) (end 97.612744 81.707) (width 1) (layer "B.Cu") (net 11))
 (segment (start 100.239438 81.620306) (end 100.239438 82.822387) (width 1) (layer "B.Cu") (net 12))
 (segment (start 97.854825 85.207) (end 94.447 85.207) (width 1) (layer "B.Cu") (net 12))
 (segment (start 100.239438 82.822387) (end 97.854825 85.207) (width 1) (layer "B.Cu") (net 12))
 (segment (start 66 68.525) (end 66 76) (width 1) (layer "F.Cu") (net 9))
 (segment (start 66 76) (end 68.3 78.3) (width 1) (layer "F.Cu") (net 9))
 (via (at 68.3 78.3) (size 1.5) (drill 0.75) (layers "F.Cu" "B.Cu") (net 9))
 (segment (start 68.3 78.3) (end 77.048 78.3) (width 1) (layer "B.Cu") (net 9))
 (segment (start 83.71 83.29) (end 83.71 60.21) (width 1) (layer "B.Cu") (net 4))
 (segment (start 75.937919 66.78) (end 73.5 64.342081) (width 1) (layer "B.Cu") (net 4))
 (segment (start 77.048 85.92) (end 81.08 85.92) (width 1) (layer "B.Cu") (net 4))
 (segment (start 73.5 64.342081) (end 73.5 57) (width 1) (layer "B.Cu") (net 4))
 (segment (start 77.14 66.78) (end 75.937919 66.78) (width 1) (layer "B.Cu") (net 4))
 (segment (start 83.71 60.21) (end 77.14 66.78) (width 1) (layer "B.Cu") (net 4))
 (segment (start 85.25 60.21) (end 87.23 58.23) (width 1) (layer "B.Cu") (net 4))
 (segment (start 103 51.725) (end 105.225 49.5) (width 1) (layer "B.Cu") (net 4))
 (segment (start 87.23 56.69) (end 87.23 58.23) (width 1) (layer "B.Cu") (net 4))
 (segment (start 68.46 51.96) (end 68.46 50) (width 1) (layer "B.Cu") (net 4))
 (segment (start 83.71 60.21) (end 85.25 60.21) (width 1) (layer "B.Cu") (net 4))
 (segment (start 81.08 85.92) (end 83.71 83.29) (width 1) (layer "B.Cu") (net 4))
 (segment (start 103 69.5) (end 103 51.725) (width 1) (layer "B.Cu") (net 4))
 (segment (start 103 69.5) (end 105 71.5) (width 1) (layer "B.Cu") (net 4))
 (segment (start 73.5 57) (end 68.46 51.96) (width 1) (layer "B.Cu") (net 4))
 (segment (start 87.23 56.69) (end 87.23 49.67) (width 1) (layer "B.Cu") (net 4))
 (segment (start 98.5 69.5) (end 103 69.5) (width 1) (layer "B.Cu") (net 4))
 (segment (start 87.23 58.23) (end 98.5 69.5) (width 1) (layer "B.Cu") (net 4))
 (segment (start 82 82.5) (end 81.12 83.38) (width 1) (layer "F.Cu") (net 10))
 (segment (start 81.12 83.38) (end 77.048 83.38) (width 1) (layer "F.Cu") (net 10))
 (segment (start 79.62 56.62) (end 82 59) (width 1) (layer "F.Cu") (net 10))
 (segment (start 82 59) (end 82 82.5) (width 1) (layer "F.Cu") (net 10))
 (segment (start 77.14 56.62) (end 79.62 56.62) (width 1) (layer "F.Cu") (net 10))
 (segment (start 102.38 56.62) (end 100 56.62) (width 1) (layer "F.Cu") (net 14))
 (segment (start 108.5 54) (end 105 54) (width 1) (layer "F.Cu") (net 14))
 (segment (start 105 54) (end 102.38 56.62) (width 1) (layer "F.Cu") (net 14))
 (segment (start 113.5 62.5) (end 113.5 68.5) (width 1) (layer "F.Cu") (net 16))
 (segment (start 101.16 58) (end 109 58) (width 1) (layer "F.Cu") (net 16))
 (segment (start 109 58) (end 113.5 62.5) (width 1) (layer "F.Cu") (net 16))
 (segment (start 100 59.16) (end 101.16 58) (width 1) (layer "F.Cu") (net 16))
 (segment (start 104.5 64.5) (end 101.7 61.7) (width 1) (layer "F.Cu") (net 15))
 (segment (start 101.7 61.7) (end 100 61.7) (width 1) (layer "F.Cu") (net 15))
 (segment (start 108.5 64.5) (end 104.5 64.5) (width 1) (layer "F.Cu") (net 15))
 (segment (start 108.5 68.5) (end 108.5 64.5) (width 1) (layer "F.Cu") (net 15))
 (segment (start 107.765 49.5) (end 106.915 50.35) (width 1) (layer "B.Cu") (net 19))
 (segment (start 105 75.31) (end 105.236 75.546) (width 1) (layer "B.Cu") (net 19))
 (segment (start 107.5 75.546) (end 114.454 75.546) (width 1) (layer "B.Cu") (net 19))
 (segment (start 115.5 74.5) (end 115.54 74.54) (width 1) (layer "B.Cu") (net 19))
 (segment (start 105.236 75.546) (end 107.5 75.546) (width 1) (layer "B.Cu") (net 19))
 (segment (start 115.54 74.54) (end 117.5 74.54) (width 1) (layer "B.Cu") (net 19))
 (segment (start 105 75.31) (end 105 74.04) (width 1) (layer "B.Cu") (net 19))
 (segment (start 106.915 50.35) (end 106.915 69.915) (width 1) (layer "B.Cu") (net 19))
 (segment (start 114.454 75.546) (end 115.5 74.5) (width 1) (layer "B.Cu") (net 19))
 (segment (start 106.915 69.915) (end 107.5 70.5) (width 1) (layer "B.Cu") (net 19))
 (segment (start 107.5 70.5) (end 107.5 75.546) (width 1) (layer "B.Cu") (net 19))
 (segment (start 89.77 51.27) (end 89.77 49.67) (width 1) (layer "F.Cu") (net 2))
 (segment (start 100 54.08) (end 92.58 54.08) (width 1) (layer "F.Cu") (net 2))
 (segment (start 92.58 54.08) (end 89.77 51.27) (width 1) (layer "F.Cu") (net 2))
 (segment (start 94.14 51.5) (end 92.31 49.67) (width 1) (layer "F.Cu") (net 3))
 (segment (start 100 51.54) (end 99.96 51.5) (width 1) (layer "F.Cu") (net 3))
 (segment (start 99.96 51.5) (end 94.14 51.5) (width 1) (layer "F.Cu") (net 3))
 (segment (start 110 71.505) (end 108.505 71.505) (width 1) (layer "F.Cu") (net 7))
 (segment (start 101.24 64.24) (end 100 64.24) (width 1) (layer "F.Cu") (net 7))
 (segment (start 108.505 71.505) (end 101.24 64.24) (width 1) (layer "F.Cu") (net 7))
 (segment (start 68.5 57.568426) (end 68.5 55) (width 1) (layer "F.Cu") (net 21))
 (segment (start 77.14 59.16) (end 76.253511 58.273511) (width 1) (layer "F.Cu") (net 21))
 (segment (start 76.253511 58.273511) (end 69.205085 58.273511) (width 1) (layer "F.Cu") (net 21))
 (segment (start 69.205085 58.273511) (end 68.5 57.568426) (width 1) (layer "F.Cu") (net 21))
 (via (at 62.25 50.5) (size 2.4) (drill 2.3) (layers "F.Cu" "B.Cu") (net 21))
 (segment (start 114.25 80.75) (end 107.75 80.75) (width 1) (layer "F.Cu") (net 5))
 (segment (start 98.793001 78) (end 105 78) (width 1) (layer "F.Cu") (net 5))
 (segment (start 93.5 72.706999) (end 98.793001 78) (width 1) (layer "F.Cu") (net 5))
 (segment (start 105 78) (end 107.75 80.75) (width 1) (layer "F.Cu") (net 5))
 (segment (start 80.08 54.08) (end 93.5 67.5) (width 1) (layer "F.Cu") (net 5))
 (segment (start 93.5 67.5) (end 93.5 72.706999) (width 1) (layer "F.Cu") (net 5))
 (segment (start 77.14 54.08) (end 80.08 54.08) (width 1) (layer "F.Cu") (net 5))
 (segment (start 73 73) (end 69.75 76.25) (width 1) (layer "F.Cu") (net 8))
 (segment (start 73 62.5) (end 73 73) (width 1) (layer "F.Cu") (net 8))
 (segment (start 77.14 61.7) (end 73.8 61.7) (width 1) (layer "F.Cu") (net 8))
 (segment (start 73.8 61.7) (end 73 62.5) (width 1) (layer "F.Cu") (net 8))
 (segment (start 69.75 76.25) (end 69.75 80.75) (width 1) (layer "F.Cu") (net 8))
 (segment (start 110 74.045) (end 110 77.46) (width 1) (layer "F.Cu") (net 6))
 (segment (start 110 77.46) (end 109.96 77.5) (width 1) (layer "F.Cu") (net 6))
 (segment (start 117.5 72) (end 112.045 72) (width 1) (layer "B.Cu") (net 6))
 (segment (start 112.045 72) (end 110 74.045) (width 1) (layer "B.Cu") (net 6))
 (segment (start 65.995001 62.995001) (end 68.5 65.5) (width 1) (layer "F.Cu") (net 13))
 (segment (start 65.995001 60) (end 65.995001 62.995001) (width 1) (layer "F.Cu") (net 13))
 (segment (start 68.5 65.5) (end 68.5 68.525) (width 1) (layer "F.Cu") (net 13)))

